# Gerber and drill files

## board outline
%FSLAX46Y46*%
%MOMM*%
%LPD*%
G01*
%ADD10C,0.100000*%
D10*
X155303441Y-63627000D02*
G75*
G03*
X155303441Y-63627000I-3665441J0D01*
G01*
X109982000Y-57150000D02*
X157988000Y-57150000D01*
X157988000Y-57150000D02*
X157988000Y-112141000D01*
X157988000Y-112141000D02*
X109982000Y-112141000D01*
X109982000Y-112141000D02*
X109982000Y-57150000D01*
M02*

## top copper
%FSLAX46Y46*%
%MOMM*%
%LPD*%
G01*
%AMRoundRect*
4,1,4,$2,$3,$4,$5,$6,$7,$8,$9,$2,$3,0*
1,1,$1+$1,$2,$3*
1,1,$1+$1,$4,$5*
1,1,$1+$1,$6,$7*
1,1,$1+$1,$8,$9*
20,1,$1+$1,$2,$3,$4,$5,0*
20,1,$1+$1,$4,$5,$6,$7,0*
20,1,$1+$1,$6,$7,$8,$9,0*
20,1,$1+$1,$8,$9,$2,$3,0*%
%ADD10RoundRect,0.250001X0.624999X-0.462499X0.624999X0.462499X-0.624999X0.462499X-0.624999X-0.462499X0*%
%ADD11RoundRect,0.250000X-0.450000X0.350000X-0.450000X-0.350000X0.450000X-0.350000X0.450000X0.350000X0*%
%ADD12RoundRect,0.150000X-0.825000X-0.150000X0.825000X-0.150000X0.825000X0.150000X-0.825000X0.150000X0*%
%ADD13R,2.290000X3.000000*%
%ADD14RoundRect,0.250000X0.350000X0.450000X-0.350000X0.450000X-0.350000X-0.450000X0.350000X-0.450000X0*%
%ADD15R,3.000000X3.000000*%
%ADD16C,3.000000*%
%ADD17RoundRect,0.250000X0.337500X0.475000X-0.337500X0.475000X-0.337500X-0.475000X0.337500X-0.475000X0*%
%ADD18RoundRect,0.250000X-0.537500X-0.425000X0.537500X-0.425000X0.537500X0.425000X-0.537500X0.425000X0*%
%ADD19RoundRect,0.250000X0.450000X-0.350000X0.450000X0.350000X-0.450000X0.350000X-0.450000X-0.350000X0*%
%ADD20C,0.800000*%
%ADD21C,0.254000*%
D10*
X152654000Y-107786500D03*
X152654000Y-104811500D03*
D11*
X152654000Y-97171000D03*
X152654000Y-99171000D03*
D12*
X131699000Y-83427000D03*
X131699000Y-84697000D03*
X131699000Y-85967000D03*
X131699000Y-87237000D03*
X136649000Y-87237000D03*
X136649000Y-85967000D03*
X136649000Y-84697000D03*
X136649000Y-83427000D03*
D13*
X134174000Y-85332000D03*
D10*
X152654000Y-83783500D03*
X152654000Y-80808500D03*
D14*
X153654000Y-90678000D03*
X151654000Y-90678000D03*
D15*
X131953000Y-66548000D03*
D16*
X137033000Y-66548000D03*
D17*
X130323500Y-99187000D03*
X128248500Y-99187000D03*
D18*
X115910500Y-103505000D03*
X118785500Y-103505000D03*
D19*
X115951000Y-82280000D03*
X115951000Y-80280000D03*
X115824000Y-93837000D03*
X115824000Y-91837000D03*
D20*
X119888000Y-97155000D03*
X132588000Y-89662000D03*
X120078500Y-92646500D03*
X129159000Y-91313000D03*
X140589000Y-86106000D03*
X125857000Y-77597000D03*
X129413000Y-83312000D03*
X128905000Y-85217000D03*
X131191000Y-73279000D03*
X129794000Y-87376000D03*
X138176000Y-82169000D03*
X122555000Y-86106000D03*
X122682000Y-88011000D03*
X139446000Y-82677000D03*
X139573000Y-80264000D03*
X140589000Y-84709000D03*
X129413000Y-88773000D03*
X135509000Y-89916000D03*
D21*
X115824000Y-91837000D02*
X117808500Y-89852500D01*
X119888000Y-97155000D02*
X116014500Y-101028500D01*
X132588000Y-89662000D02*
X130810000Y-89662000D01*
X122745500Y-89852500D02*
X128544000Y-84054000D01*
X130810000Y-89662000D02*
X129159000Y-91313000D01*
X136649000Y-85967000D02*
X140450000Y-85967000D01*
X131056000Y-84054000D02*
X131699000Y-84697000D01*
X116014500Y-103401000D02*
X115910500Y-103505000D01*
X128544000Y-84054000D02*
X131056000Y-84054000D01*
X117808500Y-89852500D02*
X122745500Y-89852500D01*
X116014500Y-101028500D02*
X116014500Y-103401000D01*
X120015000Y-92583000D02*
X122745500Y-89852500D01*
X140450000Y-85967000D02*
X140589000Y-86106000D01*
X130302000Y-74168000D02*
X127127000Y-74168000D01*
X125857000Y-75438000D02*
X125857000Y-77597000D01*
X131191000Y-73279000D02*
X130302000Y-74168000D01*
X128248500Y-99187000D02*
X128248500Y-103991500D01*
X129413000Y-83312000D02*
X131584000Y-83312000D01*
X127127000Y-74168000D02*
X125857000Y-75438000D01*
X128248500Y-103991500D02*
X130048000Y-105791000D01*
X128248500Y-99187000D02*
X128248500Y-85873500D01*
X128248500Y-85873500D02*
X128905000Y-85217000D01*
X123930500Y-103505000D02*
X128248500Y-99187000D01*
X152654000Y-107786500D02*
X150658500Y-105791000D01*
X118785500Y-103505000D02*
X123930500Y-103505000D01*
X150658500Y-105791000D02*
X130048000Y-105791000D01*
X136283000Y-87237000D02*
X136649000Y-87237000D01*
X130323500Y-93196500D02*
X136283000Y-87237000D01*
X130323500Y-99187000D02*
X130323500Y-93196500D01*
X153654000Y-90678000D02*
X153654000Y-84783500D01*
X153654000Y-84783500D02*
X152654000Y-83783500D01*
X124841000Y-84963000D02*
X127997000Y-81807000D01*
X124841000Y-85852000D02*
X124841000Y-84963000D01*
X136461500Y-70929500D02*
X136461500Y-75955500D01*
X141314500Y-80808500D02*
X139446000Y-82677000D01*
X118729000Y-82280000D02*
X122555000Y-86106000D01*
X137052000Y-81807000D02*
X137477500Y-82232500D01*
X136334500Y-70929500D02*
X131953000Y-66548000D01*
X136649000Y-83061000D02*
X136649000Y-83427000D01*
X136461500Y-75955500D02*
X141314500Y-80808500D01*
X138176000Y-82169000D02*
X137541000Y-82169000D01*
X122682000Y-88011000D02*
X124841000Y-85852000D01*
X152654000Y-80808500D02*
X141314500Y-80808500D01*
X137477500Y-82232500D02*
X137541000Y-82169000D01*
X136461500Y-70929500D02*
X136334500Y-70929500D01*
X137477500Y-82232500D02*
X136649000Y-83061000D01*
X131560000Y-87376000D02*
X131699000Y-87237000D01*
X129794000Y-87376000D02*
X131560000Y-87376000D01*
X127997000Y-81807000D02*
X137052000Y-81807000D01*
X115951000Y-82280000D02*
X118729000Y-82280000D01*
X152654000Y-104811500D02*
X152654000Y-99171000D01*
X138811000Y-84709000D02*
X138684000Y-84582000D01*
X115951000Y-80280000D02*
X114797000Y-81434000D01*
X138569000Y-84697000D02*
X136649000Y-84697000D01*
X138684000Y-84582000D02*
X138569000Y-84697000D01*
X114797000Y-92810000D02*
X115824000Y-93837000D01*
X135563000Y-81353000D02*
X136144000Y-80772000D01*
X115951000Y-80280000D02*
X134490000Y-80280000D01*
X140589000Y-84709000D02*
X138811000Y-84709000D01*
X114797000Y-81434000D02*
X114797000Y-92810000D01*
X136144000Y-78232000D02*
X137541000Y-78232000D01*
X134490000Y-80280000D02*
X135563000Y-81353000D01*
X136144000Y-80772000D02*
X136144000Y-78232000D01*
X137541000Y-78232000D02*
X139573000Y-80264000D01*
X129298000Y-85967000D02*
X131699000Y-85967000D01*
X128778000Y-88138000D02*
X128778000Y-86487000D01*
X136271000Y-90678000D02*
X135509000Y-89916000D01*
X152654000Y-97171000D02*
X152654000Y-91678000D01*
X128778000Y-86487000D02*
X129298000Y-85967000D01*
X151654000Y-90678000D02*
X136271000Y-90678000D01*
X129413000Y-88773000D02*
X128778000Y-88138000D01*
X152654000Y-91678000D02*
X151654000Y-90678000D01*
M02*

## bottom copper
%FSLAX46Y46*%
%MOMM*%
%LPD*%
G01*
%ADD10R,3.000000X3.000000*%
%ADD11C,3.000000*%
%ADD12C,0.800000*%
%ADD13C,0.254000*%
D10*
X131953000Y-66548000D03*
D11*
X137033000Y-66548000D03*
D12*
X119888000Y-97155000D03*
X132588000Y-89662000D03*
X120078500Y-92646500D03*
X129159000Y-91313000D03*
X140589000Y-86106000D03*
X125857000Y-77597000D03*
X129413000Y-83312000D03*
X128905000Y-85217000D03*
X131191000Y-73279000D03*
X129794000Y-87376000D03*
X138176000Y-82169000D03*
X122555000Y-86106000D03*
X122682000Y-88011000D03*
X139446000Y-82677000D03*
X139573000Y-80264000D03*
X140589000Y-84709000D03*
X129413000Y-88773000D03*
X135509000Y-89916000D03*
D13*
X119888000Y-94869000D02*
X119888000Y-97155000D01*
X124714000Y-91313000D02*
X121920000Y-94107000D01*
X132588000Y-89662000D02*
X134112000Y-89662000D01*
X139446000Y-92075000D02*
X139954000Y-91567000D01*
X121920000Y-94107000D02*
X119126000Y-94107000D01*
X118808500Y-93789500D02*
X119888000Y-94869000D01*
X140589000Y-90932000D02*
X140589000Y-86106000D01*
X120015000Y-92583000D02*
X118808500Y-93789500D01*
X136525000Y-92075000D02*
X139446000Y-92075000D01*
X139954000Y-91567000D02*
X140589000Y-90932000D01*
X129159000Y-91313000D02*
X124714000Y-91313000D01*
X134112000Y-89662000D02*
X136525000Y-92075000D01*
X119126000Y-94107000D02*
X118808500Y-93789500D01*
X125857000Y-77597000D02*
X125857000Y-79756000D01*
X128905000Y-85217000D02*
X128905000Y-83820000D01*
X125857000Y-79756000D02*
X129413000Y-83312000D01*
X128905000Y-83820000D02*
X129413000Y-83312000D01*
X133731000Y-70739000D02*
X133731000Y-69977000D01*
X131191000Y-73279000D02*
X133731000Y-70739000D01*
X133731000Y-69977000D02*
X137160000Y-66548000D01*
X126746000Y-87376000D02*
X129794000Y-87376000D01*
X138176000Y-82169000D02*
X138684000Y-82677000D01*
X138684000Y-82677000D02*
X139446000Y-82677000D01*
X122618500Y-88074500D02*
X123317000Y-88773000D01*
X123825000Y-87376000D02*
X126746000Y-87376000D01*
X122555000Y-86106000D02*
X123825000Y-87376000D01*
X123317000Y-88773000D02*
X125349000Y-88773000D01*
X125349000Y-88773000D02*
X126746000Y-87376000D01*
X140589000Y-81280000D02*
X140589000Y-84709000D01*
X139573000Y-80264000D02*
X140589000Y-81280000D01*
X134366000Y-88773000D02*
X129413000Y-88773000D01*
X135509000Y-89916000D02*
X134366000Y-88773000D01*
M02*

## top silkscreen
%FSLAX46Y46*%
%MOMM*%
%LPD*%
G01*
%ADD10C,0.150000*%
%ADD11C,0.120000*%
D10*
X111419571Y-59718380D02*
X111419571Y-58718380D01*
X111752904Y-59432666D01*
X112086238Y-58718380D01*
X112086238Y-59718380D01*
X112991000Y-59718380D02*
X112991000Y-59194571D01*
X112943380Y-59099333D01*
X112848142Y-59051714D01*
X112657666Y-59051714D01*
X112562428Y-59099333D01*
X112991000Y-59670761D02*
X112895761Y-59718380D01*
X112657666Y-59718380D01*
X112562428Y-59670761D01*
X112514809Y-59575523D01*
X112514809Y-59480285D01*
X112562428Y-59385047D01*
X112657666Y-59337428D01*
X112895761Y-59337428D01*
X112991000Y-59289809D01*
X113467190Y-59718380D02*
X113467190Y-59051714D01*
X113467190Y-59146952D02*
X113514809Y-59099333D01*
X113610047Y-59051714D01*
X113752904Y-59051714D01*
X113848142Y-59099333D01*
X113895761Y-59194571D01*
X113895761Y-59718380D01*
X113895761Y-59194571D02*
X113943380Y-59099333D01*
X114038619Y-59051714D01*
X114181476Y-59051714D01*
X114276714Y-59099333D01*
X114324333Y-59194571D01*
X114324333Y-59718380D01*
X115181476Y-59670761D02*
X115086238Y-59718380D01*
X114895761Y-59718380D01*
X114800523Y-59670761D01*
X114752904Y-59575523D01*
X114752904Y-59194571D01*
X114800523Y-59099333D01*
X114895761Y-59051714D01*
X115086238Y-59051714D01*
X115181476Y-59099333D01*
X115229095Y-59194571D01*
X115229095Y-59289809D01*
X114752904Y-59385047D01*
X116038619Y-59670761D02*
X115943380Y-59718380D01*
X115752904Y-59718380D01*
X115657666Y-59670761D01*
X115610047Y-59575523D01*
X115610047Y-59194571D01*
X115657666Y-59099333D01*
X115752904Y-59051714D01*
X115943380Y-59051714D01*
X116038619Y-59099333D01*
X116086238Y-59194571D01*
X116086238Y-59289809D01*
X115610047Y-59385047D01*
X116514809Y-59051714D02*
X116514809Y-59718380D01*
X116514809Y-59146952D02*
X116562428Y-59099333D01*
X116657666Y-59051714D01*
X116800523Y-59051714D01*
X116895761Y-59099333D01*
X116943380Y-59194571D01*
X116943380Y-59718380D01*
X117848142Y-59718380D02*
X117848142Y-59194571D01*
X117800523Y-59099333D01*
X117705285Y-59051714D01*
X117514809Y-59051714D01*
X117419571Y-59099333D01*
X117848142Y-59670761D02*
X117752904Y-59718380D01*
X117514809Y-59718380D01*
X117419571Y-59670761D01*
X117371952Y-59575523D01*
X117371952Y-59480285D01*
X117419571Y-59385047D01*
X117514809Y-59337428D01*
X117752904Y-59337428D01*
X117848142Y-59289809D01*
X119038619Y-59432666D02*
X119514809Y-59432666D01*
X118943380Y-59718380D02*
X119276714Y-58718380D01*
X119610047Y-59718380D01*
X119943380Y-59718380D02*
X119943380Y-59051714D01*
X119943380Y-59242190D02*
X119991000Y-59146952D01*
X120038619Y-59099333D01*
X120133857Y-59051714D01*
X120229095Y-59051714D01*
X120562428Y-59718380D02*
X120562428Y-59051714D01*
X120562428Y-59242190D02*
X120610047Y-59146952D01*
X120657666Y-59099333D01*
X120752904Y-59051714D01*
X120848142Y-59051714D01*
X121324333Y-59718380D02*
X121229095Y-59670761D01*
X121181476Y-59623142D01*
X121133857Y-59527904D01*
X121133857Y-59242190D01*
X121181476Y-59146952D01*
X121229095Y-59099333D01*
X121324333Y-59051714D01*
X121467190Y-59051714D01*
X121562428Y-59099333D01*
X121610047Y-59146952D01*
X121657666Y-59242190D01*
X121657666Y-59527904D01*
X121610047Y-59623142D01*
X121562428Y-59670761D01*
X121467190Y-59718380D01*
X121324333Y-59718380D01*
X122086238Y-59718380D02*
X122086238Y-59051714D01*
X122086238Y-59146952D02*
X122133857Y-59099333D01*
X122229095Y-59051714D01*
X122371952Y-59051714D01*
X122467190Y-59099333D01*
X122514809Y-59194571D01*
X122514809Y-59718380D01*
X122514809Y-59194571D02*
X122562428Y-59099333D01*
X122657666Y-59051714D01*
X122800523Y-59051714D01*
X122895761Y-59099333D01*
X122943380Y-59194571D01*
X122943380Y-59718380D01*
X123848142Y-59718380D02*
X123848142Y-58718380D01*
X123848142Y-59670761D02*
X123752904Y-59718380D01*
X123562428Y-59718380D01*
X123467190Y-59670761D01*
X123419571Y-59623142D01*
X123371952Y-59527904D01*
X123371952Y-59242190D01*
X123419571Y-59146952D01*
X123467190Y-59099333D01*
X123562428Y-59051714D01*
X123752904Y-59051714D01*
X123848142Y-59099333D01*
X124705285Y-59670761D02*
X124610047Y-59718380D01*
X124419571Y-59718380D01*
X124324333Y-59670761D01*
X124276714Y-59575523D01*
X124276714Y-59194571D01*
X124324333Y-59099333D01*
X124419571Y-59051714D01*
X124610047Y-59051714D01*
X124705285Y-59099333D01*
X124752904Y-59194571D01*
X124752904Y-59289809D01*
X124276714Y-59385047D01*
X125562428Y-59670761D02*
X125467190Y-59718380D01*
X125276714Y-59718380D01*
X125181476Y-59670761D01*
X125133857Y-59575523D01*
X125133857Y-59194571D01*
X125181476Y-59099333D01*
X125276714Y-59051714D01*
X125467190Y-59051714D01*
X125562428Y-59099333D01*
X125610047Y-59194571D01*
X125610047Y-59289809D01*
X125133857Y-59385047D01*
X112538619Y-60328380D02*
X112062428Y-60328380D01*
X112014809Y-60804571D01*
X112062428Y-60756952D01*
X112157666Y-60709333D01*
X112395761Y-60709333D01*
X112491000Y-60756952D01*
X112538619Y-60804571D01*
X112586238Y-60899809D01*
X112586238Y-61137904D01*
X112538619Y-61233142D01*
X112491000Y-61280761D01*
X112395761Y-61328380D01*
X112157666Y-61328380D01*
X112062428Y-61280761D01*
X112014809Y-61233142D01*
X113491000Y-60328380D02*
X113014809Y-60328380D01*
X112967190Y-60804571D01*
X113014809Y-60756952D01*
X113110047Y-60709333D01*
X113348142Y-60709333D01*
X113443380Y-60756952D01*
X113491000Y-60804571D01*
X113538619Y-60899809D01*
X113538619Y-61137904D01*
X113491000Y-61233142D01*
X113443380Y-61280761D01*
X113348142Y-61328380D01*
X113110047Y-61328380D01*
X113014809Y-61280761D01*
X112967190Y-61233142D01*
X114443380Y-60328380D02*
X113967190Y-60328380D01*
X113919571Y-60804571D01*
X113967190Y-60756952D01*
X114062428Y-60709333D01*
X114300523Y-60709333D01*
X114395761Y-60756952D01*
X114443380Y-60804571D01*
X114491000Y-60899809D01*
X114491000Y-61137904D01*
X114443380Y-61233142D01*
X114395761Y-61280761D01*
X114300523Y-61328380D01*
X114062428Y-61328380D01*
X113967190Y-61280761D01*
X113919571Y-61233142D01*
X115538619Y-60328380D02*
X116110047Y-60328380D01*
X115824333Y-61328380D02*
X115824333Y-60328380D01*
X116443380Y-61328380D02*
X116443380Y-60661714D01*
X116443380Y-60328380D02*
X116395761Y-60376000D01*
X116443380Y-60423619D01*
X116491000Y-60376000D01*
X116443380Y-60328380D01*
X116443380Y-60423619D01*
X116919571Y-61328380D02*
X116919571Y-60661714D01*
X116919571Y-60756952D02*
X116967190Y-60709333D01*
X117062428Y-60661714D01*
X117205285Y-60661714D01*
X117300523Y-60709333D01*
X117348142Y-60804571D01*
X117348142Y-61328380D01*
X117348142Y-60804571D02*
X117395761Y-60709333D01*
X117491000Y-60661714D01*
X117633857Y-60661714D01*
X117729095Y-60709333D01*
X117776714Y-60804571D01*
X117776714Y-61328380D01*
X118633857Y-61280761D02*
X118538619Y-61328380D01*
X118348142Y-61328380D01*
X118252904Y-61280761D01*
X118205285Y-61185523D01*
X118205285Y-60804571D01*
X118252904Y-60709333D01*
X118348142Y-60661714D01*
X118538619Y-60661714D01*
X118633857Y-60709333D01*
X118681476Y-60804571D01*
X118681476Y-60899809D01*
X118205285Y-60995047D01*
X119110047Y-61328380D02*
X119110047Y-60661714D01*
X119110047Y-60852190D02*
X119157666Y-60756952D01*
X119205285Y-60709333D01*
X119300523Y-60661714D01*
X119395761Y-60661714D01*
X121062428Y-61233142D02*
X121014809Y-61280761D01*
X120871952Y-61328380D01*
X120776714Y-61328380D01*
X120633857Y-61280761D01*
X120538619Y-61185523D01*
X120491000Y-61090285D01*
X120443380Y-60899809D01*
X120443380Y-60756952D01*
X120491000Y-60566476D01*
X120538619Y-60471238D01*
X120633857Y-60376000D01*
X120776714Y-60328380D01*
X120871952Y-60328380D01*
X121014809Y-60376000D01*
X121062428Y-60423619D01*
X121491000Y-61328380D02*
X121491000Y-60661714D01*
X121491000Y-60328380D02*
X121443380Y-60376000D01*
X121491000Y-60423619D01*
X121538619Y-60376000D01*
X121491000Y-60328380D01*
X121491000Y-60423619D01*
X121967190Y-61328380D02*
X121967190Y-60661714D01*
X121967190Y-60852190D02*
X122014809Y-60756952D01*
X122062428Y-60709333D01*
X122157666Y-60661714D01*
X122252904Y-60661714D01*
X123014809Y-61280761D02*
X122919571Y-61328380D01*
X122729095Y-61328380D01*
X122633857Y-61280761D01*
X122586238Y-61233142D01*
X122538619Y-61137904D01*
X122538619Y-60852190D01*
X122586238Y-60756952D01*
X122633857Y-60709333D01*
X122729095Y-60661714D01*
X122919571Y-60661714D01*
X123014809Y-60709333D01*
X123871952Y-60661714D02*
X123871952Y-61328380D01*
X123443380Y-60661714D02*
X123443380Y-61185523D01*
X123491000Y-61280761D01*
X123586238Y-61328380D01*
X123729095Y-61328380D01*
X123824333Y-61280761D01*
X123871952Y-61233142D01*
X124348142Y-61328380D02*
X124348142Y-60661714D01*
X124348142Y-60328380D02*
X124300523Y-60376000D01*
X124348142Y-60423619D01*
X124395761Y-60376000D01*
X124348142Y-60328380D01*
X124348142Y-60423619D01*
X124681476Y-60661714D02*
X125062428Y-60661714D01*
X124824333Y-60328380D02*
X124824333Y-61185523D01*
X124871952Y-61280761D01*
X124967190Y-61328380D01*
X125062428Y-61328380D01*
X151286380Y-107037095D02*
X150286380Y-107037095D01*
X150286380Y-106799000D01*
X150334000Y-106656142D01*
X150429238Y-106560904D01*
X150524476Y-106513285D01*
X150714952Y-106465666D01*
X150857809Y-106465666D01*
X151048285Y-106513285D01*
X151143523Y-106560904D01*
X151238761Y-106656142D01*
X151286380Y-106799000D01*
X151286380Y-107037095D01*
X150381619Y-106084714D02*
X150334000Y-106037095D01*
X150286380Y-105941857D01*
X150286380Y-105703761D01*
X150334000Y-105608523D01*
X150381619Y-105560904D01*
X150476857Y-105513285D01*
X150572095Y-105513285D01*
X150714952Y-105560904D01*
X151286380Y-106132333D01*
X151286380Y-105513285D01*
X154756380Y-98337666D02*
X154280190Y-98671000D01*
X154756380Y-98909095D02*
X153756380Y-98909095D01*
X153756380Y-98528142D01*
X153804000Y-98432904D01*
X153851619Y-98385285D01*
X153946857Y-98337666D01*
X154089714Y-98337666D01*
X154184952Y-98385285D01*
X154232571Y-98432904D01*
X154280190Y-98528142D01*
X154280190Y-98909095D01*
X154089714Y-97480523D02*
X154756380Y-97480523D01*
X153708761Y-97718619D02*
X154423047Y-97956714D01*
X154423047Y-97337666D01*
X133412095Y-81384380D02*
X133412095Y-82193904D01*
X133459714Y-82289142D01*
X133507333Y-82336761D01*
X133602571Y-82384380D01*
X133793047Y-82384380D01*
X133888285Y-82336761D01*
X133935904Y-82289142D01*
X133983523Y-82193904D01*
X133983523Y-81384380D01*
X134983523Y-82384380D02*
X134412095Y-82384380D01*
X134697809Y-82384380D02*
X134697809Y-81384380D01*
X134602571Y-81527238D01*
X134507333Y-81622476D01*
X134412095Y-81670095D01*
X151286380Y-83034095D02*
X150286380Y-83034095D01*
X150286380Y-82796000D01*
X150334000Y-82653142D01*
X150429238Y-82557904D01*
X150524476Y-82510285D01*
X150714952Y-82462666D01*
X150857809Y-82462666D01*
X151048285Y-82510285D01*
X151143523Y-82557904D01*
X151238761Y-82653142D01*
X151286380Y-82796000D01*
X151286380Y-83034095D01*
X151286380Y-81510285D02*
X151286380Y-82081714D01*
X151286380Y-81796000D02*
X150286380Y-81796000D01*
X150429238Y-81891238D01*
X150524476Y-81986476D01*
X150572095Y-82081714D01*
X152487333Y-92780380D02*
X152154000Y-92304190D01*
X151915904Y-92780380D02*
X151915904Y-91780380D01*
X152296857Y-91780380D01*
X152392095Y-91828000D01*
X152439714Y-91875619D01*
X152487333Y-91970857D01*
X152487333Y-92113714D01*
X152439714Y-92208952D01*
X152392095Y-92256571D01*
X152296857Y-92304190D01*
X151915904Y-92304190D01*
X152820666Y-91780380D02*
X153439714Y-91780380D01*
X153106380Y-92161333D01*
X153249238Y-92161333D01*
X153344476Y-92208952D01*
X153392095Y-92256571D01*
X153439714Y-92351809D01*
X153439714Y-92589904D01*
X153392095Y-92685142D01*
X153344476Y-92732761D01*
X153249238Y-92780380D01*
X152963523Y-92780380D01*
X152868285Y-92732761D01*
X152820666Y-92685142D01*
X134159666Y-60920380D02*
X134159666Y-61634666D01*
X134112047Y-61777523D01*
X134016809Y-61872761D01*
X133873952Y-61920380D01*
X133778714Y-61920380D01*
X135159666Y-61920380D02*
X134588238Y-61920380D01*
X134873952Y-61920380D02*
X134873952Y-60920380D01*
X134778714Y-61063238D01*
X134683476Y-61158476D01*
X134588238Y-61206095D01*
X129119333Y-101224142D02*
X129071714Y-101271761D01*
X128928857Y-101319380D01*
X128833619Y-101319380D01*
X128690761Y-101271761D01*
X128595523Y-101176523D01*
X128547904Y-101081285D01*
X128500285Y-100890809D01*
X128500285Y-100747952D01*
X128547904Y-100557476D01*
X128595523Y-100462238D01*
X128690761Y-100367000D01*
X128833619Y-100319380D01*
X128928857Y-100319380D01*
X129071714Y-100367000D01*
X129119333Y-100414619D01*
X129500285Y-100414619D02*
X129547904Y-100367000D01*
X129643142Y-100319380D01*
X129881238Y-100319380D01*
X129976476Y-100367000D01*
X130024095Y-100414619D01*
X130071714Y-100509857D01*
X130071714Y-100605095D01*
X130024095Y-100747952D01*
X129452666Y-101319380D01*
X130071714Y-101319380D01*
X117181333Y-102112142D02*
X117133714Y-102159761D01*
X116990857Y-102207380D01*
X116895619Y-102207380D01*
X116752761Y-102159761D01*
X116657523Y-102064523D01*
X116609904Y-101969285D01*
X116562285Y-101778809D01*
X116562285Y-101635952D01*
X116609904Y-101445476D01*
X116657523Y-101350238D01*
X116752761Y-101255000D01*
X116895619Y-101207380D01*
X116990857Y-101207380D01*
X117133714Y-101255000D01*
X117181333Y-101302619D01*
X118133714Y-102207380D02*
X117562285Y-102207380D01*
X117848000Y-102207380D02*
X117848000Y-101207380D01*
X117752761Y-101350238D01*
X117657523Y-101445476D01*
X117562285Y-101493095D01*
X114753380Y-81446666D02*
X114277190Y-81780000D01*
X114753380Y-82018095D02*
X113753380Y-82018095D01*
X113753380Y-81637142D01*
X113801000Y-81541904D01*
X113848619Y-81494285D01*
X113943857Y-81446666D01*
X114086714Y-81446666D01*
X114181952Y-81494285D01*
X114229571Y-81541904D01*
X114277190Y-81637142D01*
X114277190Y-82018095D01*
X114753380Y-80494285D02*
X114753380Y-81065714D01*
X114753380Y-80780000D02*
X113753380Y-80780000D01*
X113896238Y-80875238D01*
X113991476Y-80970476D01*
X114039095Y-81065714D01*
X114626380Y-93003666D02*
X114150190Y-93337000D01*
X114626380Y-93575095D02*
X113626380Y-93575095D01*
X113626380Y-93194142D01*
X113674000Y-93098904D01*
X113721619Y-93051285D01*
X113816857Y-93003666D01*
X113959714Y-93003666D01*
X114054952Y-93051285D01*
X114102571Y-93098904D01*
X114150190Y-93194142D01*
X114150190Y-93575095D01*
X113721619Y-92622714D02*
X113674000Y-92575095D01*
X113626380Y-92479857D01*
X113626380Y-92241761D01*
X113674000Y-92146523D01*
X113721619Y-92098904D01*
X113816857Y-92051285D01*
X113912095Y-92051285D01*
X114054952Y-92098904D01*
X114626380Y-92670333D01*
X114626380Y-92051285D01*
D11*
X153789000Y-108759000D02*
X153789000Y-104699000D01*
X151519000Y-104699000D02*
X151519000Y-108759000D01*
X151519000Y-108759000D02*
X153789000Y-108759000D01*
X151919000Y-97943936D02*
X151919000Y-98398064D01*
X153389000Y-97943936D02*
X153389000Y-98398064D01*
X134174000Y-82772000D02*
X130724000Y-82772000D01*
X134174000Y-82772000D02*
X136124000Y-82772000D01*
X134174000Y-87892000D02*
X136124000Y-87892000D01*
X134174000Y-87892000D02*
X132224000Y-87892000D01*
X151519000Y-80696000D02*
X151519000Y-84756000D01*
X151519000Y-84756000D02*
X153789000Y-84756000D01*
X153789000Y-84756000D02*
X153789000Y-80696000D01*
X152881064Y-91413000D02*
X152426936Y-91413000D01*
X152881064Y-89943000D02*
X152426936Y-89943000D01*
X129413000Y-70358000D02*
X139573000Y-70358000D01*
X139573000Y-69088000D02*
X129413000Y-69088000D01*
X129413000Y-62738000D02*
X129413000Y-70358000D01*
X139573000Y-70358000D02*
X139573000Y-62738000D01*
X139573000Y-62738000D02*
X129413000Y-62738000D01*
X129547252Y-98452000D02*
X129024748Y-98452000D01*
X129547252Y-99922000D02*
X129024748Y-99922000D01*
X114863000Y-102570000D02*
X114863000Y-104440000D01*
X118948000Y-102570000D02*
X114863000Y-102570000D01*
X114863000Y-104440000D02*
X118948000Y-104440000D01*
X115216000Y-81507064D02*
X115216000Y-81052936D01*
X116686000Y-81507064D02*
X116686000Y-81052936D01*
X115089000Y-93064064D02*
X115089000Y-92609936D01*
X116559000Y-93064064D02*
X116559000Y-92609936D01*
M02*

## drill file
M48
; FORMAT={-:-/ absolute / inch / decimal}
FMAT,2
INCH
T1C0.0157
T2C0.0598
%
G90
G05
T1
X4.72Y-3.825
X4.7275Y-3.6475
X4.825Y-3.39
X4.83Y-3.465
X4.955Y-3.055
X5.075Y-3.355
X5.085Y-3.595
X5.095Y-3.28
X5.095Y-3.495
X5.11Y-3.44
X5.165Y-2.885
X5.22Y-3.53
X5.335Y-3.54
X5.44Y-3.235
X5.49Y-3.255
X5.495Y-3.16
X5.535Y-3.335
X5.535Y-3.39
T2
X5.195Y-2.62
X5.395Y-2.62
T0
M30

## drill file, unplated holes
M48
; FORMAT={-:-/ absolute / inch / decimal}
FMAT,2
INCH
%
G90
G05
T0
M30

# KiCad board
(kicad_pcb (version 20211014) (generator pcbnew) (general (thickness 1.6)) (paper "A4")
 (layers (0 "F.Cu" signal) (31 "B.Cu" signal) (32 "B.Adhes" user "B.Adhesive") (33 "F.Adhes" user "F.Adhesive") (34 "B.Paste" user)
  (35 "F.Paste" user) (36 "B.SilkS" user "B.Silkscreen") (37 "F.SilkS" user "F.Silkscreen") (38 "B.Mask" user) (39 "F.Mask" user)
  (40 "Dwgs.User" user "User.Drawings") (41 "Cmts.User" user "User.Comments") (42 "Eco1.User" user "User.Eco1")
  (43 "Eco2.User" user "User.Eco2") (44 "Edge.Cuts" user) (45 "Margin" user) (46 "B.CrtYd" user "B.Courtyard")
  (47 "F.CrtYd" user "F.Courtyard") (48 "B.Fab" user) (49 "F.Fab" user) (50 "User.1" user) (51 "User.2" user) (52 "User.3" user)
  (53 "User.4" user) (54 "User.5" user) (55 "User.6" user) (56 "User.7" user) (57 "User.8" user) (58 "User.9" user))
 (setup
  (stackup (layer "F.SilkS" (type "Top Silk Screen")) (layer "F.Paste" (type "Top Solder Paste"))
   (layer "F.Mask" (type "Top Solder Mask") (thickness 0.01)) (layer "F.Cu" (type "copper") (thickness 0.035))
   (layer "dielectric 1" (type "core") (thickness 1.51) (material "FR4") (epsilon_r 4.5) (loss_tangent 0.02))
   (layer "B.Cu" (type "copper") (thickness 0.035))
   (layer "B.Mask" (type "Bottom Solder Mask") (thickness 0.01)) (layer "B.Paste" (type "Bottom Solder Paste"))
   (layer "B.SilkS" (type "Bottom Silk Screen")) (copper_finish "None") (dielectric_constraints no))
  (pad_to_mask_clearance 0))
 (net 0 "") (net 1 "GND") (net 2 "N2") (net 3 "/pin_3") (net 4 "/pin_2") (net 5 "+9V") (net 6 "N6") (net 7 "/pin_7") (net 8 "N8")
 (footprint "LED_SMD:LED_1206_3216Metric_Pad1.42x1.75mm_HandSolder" (layer "F.Cu") (at 152.654 106.299 90)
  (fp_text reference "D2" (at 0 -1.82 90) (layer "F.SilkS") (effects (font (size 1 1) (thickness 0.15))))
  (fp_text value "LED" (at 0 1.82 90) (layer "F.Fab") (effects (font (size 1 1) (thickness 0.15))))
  (fp_line (start -2.46 1.135) (end 1.6 1.135) (layer "F.SilkS") (width 0.12))
  (fp_line (start 1.6 -1.135) (end -2.46 -1.135) (layer "F.SilkS") (width 0.12))
  (fp_line (start -2.46 -1.135) (end -2.46 1.135) (layer "F.SilkS") (width 0.12))
  (pad "1" smd roundrect (at -1.4875 0 90) (size 1.425 1.75) (layers "F.Cu" "F.Paste" "F.Mask") (roundrect_rratio 0.1754392982)
   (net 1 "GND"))
  (pad "2" smd roundrect (at 1.4875 0 90) (size 1.425 1.75) (layers "F.Cu" "F.Paste" "F.Mask") (roundrect_rratio 0.1754392982) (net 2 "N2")))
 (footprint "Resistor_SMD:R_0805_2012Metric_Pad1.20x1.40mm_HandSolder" (layer "F.Cu") (at 152.654 98.171 -90)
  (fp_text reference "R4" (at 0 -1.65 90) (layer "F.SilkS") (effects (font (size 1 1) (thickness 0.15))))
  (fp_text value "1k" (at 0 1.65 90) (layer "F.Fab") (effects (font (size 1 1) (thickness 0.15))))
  (fp_line (start -0.227064 0.735) (end 0.227064 0.735) (layer "F.SilkS") (width 0.12))
  (fp_line (start -0.227064 -0.735) (end 0.227064 -0.735) (layer "F.SilkS") (width 0.12))
  (pad "1" smd roundrect (at -1 0 270) (size 1.2 1.4) (layers "F.Cu" "F.Paste" "F.Mask") (roundrect_rratio 0.2083333333) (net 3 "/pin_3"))
  (pad "2" smd roundrect (at 1 0 270) (size 1.2 1.4) (layers "F.Cu" "F.Paste" "F.Mask") (roundrect_rratio 0.2083333333) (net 2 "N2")))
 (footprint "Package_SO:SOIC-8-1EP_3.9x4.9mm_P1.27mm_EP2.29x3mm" (layer "F.Cu") (at 134.174 85.332)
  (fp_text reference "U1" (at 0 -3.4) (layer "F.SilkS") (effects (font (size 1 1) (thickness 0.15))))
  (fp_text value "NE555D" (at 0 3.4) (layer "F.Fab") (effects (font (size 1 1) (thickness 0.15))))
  (fp_line (start 0 -2.56) (end -3.45 -2.56) (layer "F.SilkS") (width 0.12))
  (fp_line (start 0 -2.56) (end 1.95 -2.56) (layer "F.SilkS") (width 0.12))
  (fp_line (start 0 2.56) (end 1.95 2.56) (layer "F.SilkS") (width 0.12))
  (fp_line (start 0 2.56) (end -1.95 2.56) (layer "F.SilkS") (width 0.12))
  (pad "" smd roundrect (at 0.57 -0.75) (size 0.92 1.21) (layers "F.Paste") (roundrect_rratio 0.25))
  (pad "" smd roundrect (at -0.57 -0.75) (size 0.92 1.21) (layers "F.Paste") (roundrect_rratio 0.25))
  (pad "" smd roundrect (at -0.57 0.75) (size 0.92 1.21) (layers "F.Paste") (roundrect_rratio 0.25))
  (pad "" smd roundrect (at 0.57 0.75) (size 0.92 1.21) (layers "F.Paste") (roundrect_rratio 0.25))
  (pad "1" smd roundrect (at -2.475 -1.905) (size 1.95 0.6) (layers "F.Cu" "F.Paste" "F.Mask") (roundrect_rratio 0.25) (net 1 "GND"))
  (pad "2" smd roundrect (at -2.475 -0.635) (size 1.95 0.6) (layers "F.Cu" "F.Paste" "F.Mask") (roundrect_rratio 0.25) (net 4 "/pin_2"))
  (pad "3" smd roundrect (at -2.475 0.635) (size 1.95 0.6) (layers "F.Cu" "F.Paste" "F.Mask") (roundrect_rratio 0.25) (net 3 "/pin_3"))
  (pad "4" smd roundrect (at -2.475 1.905) (size 1.95 0.6) (layers "F.Cu" "F.Paste" "F.Mask") (roundrect_rratio 0.25) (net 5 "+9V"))
  (pad "5" smd roundrect (at 2.475 1.905) (size 1.95 0.6) (layers "F.Cu" "F.Paste" "F.Mask") (roundrect_rratio 0.25) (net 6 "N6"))
  (pad "6" smd roundrect (at 2.475 0.635) (size 1.95 0.6) (layers "F.Cu" "F.Paste" "F.Mask") (roundrect_rratio 0.25) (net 4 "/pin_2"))
  (pad "7" smd roundrect (at 2.475 -0.635) (size 1.95 0.6) (layers "F.Cu" "F.Paste" "F.Mask") (roundrect_rratio 0.25) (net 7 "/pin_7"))
  (pad "8" smd roundrect (at 2.475 -1.905) (size 1.95 0.6) (layers "F.Cu" "F.Paste" "F.Mask") (roundrect_rratio 0.25) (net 5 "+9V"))
  (pad "9" smd rect (at 0 0) (size 2.29 3) (layers "F.Cu" "F.Mask")))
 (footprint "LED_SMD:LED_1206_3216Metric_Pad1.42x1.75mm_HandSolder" (layer "F.Cu") (at 152.654 82.296 90)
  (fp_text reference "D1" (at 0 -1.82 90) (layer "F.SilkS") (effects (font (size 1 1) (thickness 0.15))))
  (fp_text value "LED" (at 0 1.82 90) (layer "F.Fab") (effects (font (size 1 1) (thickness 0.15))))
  (fp_line (start 1.6 -1.135) (end -2.46 -1.135) (layer "F.SilkS") (width 0.12))
  (fp_line (start -2.46 -1.135) (end -2.46 1.135) (layer "F.SilkS") (width 0.12))
  (fp_line (start -2.46 1.135) (end 1.6 1.135) (layer "F.SilkS") (width 0.12))
  (pad "1" smd roundrect (at -1.4875 0 90) (size 1.425 1.75) (layers "F.Cu" "F.Paste" "F.Mask") (roundrect_rratio 0.1754392982) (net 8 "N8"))
  (pad "2" smd roundrect (at 1.4875 0 90) (size 1.425 1.75) (layers "F.Cu" "F.Paste" "F.Mask") (roundrect_rratio 0.1754392982) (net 5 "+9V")))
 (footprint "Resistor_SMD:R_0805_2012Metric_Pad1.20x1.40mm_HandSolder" (layer "F.Cu") (at 152.654 90.678 180)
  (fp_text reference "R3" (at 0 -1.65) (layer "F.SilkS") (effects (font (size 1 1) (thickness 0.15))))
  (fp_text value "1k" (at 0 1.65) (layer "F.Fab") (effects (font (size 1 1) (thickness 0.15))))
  (fp_line (start -0.227064 -0.735) (end 0.227064 -0.735) (layer "F.SilkS") (width 0.12))
  (fp_line (start -0.227064 0.735) (end 0.227064 0.735) (layer "F.SilkS") (width 0.12))
  (pad "1" smd roundrect (at -1 0 180) (size 1.2 1.4) (layers "F.Cu" "F.Paste" "F.Mask") (roundrect_rratio 0.2083333333) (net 8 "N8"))
  (pad "2" smd roundrect (at 1 0 180) (size 1.2 1.4) (layers "F.Cu" "F.Paste" "F.Mask") (roundrect_rratio 0.2083333333) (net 3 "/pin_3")))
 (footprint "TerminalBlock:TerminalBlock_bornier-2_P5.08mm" (layer "F.Cu") (at 131.953 66.548)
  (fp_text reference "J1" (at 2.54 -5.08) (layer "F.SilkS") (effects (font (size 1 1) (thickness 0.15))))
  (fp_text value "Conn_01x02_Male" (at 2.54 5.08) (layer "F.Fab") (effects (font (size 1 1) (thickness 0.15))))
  (fp_line (start -2.54 3.81) (end 7.62 3.81) (layer "F.SilkS") (width 0.12))
  (fp_line (start 7.62 2.54) (end -2.54 2.54) (layer "F.SilkS") (width 0.12))
  (fp_line (start -2.54 -3.81) (end -2.54 3.81) (layer "F.SilkS") (width 0.12))
  (fp_line (start 7.62 3.81) (end 7.62 -3.81) (layer "F.SilkS") (width 0.12))
  (fp_line (start 7.62 -3.81) (end -2.54 -3.81) (layer "F.SilkS") (width 0.12))
  (pad "1" thru_hole rect (at 0 0) (size 3 3) (drill 1.52) (layers *.Cu *.Mask) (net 5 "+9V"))
  (pad "2" thru_hole circle (at 5.08 0) (size 3 3) (drill 1.52) (layers *.Cu *.Mask) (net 1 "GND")))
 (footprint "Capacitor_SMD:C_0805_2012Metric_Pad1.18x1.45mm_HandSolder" (layer "F.Cu") (at 129.286 99.187 180)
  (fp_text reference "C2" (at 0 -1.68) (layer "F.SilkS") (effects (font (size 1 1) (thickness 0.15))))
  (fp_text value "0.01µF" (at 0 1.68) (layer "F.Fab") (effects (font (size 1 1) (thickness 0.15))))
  (fp_line (start -0.261252 0.735) (end 0.261252 0.735) (layer "F.SilkS") (width 0.12))
  (fp_line (start -0.261252 -0.735) (end 0.261252 -0.735) (layer "F.SilkS") (width 0.12))
  (pad "1" smd roundrect (at -1.0375 0 180) (size 1.175 1.45) (layers "F.Cu" "F.Paste" "F.Mask") (roundrect_rratio 0.2127659574)
   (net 6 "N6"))
  (pad "2" smd roundrect (at 1.0375 0 180) (size 1.175 1.45) (layers "F.Cu" "F.Paste" "F.Mask") (roundrect_rratio 0.2127659574)
   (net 1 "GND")))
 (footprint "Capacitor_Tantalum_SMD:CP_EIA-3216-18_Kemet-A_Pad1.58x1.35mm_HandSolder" (layer "F.Cu") (at 117.348 103.505)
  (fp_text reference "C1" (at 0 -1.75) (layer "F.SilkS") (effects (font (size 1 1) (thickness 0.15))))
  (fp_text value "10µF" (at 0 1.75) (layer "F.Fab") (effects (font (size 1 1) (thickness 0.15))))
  (fp_line (start -2.485 -0.935) (end -2.485 0.935) (layer "F.SilkS") (width 0.12))
  (fp_line (start 1.6 -0.935) (end -2.485 -0.935) (layer "F.SilkS") (width 0.12))
  (fp_line (start -2.485 0.935) (end 1.6 0.935) (layer "F.SilkS") (width 0.12))
  (pad "1" smd roundrect (at -1.4375 0) (size 1.575 1.35) (layers "F.Cu" "F.Paste" "F.Mask") (roundrect_rratio 0.1851851852)
   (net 4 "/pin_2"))
  (pad "2" smd roundrect (at 1.4375 0) (size 1.575 1.35) (layers "F.Cu" "F.Paste" "F.Mask") (roundrect_rratio 0.1851851852) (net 1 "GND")))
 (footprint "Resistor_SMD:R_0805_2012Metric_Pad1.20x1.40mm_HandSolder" (layer "F.Cu") (at 115.951 81.28 90)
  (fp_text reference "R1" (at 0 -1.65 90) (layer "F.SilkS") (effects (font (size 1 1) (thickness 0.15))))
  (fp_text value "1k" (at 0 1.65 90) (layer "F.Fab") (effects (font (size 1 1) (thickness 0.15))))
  (fp_line (start -0.227064 -0.735) (end 0.227064 -0.735) (layer "F.SilkS") (width 0.12))
  (fp_line (start -0.227064 0.735) (end 0.227064 0.735) (layer "F.SilkS") (width 0.12))
  (pad "1" smd roundrect (at -1 0 90) (size 1.2 1.4) (layers "F.Cu" "F.Paste" "F.Mask") (roundrect_rratio 0.2083333333) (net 5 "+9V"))
  (pad "2" smd roundrect (at 1 0 90) (size 1.2 1.4) (layers "F.Cu" "F.Paste" "F.Mask") (roundrect_rratio 0.2083333333) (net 7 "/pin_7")))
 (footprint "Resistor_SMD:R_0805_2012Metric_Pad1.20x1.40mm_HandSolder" (layer "F.Cu") (at 115.824 92.837 90)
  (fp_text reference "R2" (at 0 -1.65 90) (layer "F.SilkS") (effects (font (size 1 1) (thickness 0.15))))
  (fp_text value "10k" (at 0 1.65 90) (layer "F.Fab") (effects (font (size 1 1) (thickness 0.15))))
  (fp_line (start -0.227064 -0.735) (end 0.227064 -0.735) (layer "F.SilkS") (width 0.12))
  (fp_line (start -0.227064 0.735) (end 0.227064 0.735) (layer "F.SilkS") (width 0.12))
  (pad "1" smd roundrect (at -1 0 90) (size 1.2 1.4) (layers "F.Cu" "F.Paste" "F.Mask") (roundrect_rratio 0.2083333333) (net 7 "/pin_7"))
  (pad "2" smd roundrect (at 1 0 90) (size 1.2 1.4) (layers "F.Cu" "F.Paste" "F.Mask") (roundrect_rratio 0.2083333333) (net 4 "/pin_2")))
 (gr_circle (center 151.638 63.627) (end 152.527 60.071) (layer "Edge.Cuts") (width 0.1) (fill none))
 (gr_rect (start 109.982 57.15) (end 157.988 112.141) (layer "Edge.Cuts") (width 0.1) (fill none))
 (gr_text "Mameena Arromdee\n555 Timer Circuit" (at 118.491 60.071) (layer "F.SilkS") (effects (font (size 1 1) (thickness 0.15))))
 (segment (start 115.824 91.837) (end 117.8085 89.8525) (width 0.254) (layer "F.Cu") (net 4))
 (segment (start 119.888 97.155) (end 116.0145 101.0285) (width 0.254) (layer "F.Cu") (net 4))
 (segment (start 132.588 89.662) (end 130.81 89.662) (width 0.254) (layer "F.Cu") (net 4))
 (segment (start 122.7455 89.8525) (end 128.544 84.054) (width 0.254) (layer "F.Cu") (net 4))
 (segment (start 130.81 89.662) (end 129.159 91.313) (width 0.254) (layer "F.Cu") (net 4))
 (segment (start 136.649 85.967) (end 140.45 85.967) (width 0.254) (layer "F.Cu") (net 4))
 (segment (start 131.056 84.054) (end 131.699 84.697) (width 0.254) (layer "F.Cu") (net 4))
 (segment (start 116.0145 103.401) (end 115.9105 103.505) (width 0.254) (layer "F.Cu") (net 4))
 (segment (start 128.544 84.054) (end 131.056 84.054) (width 0.254) (layer "F.Cu") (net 4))
 (segment (start 117.8085 89.8525) (end 122.7455 89.8525) (width 0.254) (layer "F.Cu") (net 4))
 (segment (start 116.0145 101.0285) (end 116.0145 103.401) (width 0.254) (layer "F.Cu") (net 4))
 (segment (start 120.015 92.583) (end 122.7455 89.8525) (width 0.254) (layer "F.Cu") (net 4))
 (segment (start 140.45 85.967) (end 140.589 86.106) (width 0.254) (layer "F.Cu") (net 4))
 (via (at 119.888 97.155) (size 0.8) (drill 0.4) (layers "F.Cu" "B.Cu") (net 4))
 (via (at 132.588 89.662) (size 0.8) (drill 0.4) (layers "F.Cu" "B.Cu") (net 4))
 (via (at 120.0785 92.6465) (size 0.8) (drill 0.4) (layers "F.Cu" "B.Cu") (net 4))
 (via (at 129.159 91.313) (size 0.8) (drill 0.4) (layers "F.Cu" "B.Cu") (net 4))
 (via (at 140.589 86.106) (size 0.8) (drill 0.4) (layers "F.Cu" "B.Cu") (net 4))
 (segment (start 119.888 94.869) (end 119.888 97.155) (width 0.254) (layer "B.Cu") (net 4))
 (segment (start 124.714 91.313) (end 121.92 94.107) (width 0.254) (layer "B.Cu") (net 4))
 (segment (start 132.588 89.662) (end 134.112 89.662) (width 0.254) (layer "B.Cu") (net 4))
 (segment (start 139.446 92.075) (end 139.954 91.567) (width 0.254) (layer "B.Cu") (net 4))
 (segment (start 121.92 94.107) (end 119.126 94.107) (width 0.254) (layer "B.Cu") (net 4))
 (segment (start 118.8085 93.7895) (end 119.888 94.869) (width 0.254) (layer "B.Cu") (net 4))
 (segment (start 140.589 90.932) (end 140.589 86.106) (width 0.254) (layer "B.Cu") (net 4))
 (segment (start 120.015 92.583) (end 118.8085 93.7895) (width 0.254) (layer "B.Cu") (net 4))
 (segment (start 136.525 92.075) (end 139.446 92.075) (width 0.254) (layer "B.Cu") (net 4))
 (segment (start 139.954 91.567) (end 140.589 90.932) (width 0.254) (layer "B.Cu") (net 4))
 (segment (start 129.159 91.313) (end 124.714 91.313) (width 0.254) (layer "B.Cu") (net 4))
 (segment (start 134.112 89.662) (end 136.525 92.075) (width 0.254) (layer "B.Cu") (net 4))
 (segment (start 119.126 94.107) (end 118.8085 93.7895) (width 0.254) (layer "B.Cu") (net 4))
 (segment (start 130.302 74.168) (end 127.127 74.168) (width 0.254) (layer "F.Cu") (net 1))
 (segment (start 125.857 75.438) (end 125.857 77.597) (width 0.254) (layer "F.Cu") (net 1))
 (segment (start 131.191 73.279) (end 130.302 74.168) (width 0.254) (layer "F.Cu") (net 1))
 (segment (start 128.2485 99.187) (end 128.2485 103.9915) (width 0.254) (layer "F.Cu") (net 1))
 (segment (start 129.413 83.312) (end 131.584 83.312) (width 0.254) (layer "F.Cu") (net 1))
 (segment (start 127.127 74.168) (end 125.857 75.438) (width 0.254) (layer "F.Cu") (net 1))
 (segment (start 128.2485 103.9915) (end 130.048 105.791) (width 0.254) (layer "F.Cu") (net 1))
 (segment (start 128.2485 99.187) (end 128.2485 85.8735) (width 0.254) (layer "F.Cu") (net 1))
 (segment (start 128.2485 85.8735) (end 128.905 85.217) (width 0.254) (layer "F.Cu") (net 1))
 (segment (start 123.9305 103.505) (end 128.2485 99.187) (width 0.254) (layer "F.Cu") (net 1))
 (segment (start 152.654 107.7865) (end 150.6585 105.791) (width 0.254) (layer "F.Cu") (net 1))
 (segment (start 118.7855 103.505) (end 123.9305 103.505) (width 0.254) (layer "F.Cu") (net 1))
 (segment (start 150.6585 105.791) (end 130.048 105.791) (width 0.254) (layer "F.Cu") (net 1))
 (via (at 125.857 77.597) (size 0.8) (drill 0.4) (layers "F.Cu" "B.Cu") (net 1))
 (via (at 129.413 83.312) (size 0.8) (drill 0.4) (layers "F.Cu" "B.Cu") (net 1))
 (via (at 128.905 85.217) (size 0.8) (drill 0.4) (layers "F.Cu" "B.Cu") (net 1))
 (via (at 131.191 73.279) (size 0.8) (drill 0.4) (layers "F.Cu" "B.Cu") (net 1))
 (segment (start 125.857 77.597) (end 125.857 79.756) (width 0.254) (layer "B.Cu") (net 1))
 (segment (start 128.905 85.217) (end 128.905 83.82) (width 0.254) (layer "B.Cu") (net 1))
 (segment (start 125.857 79.756) (end 129.413 83.312) (width 0.254) (layer "B.Cu") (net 1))
 (segment (start 128.905 83.82) (end 129.413 83.312) (width 0.254) (layer "B.Cu") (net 1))
 (segment (start 133.731 70.739) (end 133.731 69.977) (width 0.254) (layer "B.Cu") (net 1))
 (segment (start 131.191 73.279) (end 133.731 70.739) (width 0.254) (layer "B.Cu") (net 1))
 (segment (start 133.731 69.977) (end 137.16 66.548) (width 0.254) (layer "B.Cu") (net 1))
 (segment (start 136.283 87.237) (end 136.649 87.237) (width 0.254) (layer "F.Cu") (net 6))
 (segment (start 130.3235 93.1965) (end 136.283 87.237) (width 0.254) (layer "F.Cu") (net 6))
 (segment (start 130.3235 99.187) (end 130.3235 93.1965) (width 0.254) (layer "F.Cu") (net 6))
 (segment (start 153.654 90.678) (end 153.654 84.7835) (width 0.254) (layer "F.Cu") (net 8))
 (segment (start 153.654 84.7835) (end 152.654 83.7835) (width 0.254) (layer "F.Cu") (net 8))
 (segment (start 124.841 84.963) (end 127.997 81.807) (width 0.254) (layer "F.Cu") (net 5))
 (segment (start 124.841 85.852) (end 124.841 84.963) (width 0.254) (layer "F.Cu") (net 5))
 (segment (start 136.4615 70.9295) (end 136.4615 75.9555) (width 0.254) (layer "F.Cu") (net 5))
 (segment (start 141.3145 80.8085) (end 139.446 82.677) (width 0.254) (layer "F.Cu") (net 5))
 (segment (start 118.729 82.28) (end 122.555 86.106) (width 0.254) (layer "F.Cu") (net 5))
 (segment (start 137.052 81.807) (end 137.4775 82.2325) (width 0.254) (layer "F.Cu") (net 5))
 (segment (start 136.3345 70.9295) (end 131.953 66.548) (width 0.254) (layer "F.Cu") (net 5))
 (segment (start 136.649 83.061) (end 136.649 83.427) (width 0.254) (layer "F.Cu") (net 5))
 (segment (start 136.4615 75.9555) (end 141.3145 80.8085) (width 0.254) (layer "F.Cu") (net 5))
 (segment (start 138.176 82.169) (end 137.541 82.169) (width 0.254) (layer "F.Cu") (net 5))
 (segment (start 122.682 88.011) (end 124.841 85.852) (width 0.254) (layer "F.Cu") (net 5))
 (segment (start 152.654 80.8085) (end 141.3145 80.8085) (width 0.254) (layer "F.Cu") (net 5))
 (segment (start 137.4775 82.2325) (end 137.541 82.169) (width 0.254) (layer "F.Cu") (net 5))
 (segment (start 136.4615 70.9295) (end 136.3345 70.9295) (width 0.254) (layer "F.Cu") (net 5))
 (segment (start 137.4775 82.2325) (end 136.649 83.061) (width 0.254) (layer "F.Cu") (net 5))
 (segment (start 131.56 87.376) (end 131.699 87.237) (width 0.254) (layer "F.Cu") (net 5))
 (segment (start 129.794 87.376) (end 131.56 87.376) (width 0.254) (layer "F.Cu") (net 5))
 (segment (start 127.997 81.807) (end 137.052 81.807) (width 0.254) (layer "F.Cu") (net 5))
 (segment (start 115.951 82.28) (end 118.729 82.28) (width 0.254) (layer "F.Cu") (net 5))
 (via (at 129.794 87.376) (size 0.8) (drill 0.4) (layers "F.Cu" "B.Cu") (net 5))
 (via (at 138.176 82.169) (size 0.8) (drill 0.4) (layers "F.Cu" "B.Cu") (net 5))
 (via (at 122.555 86.106) (size 0.8) (drill 0.4) (layers "F.Cu" "B.Cu") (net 5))
 (via (at 122.682 88.011) (size 0.8) (drill 0.4) (layers "F.Cu" "B.Cu") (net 5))
 (via (at 139.446 82.677) (size 0.8) (drill 0.4) (layers "F.Cu" "B.Cu") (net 5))
 (segment (start 126.746 87.376) (end 129.794 87.376) (width 0.254) (layer "B.Cu") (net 5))
 (segment (start 138.176 82.169) (end 138.684 82.677) (width 0.254) (layer "B.Cu") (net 5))
 (segment (start 138.684 82.677) (end 139.446 82.677) (width 0.254) (layer "B.Cu") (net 5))
 (segment (start 122.6185 88.0745) (end 123.317 88.773) (width 0.254) (layer "B.Cu") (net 5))
 (segment (start 123.825 87.376) (end 126.746 87.376) (width 0.254) (layer "B.Cu") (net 5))
 (segment (start 122.555 86.106) (end 123.825 87.376) (width 0.254) (layer "B.Cu") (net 5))
 (segment (start 123.317 88.773) (end 125.349 88.773) (width 0.254) (layer "B.Cu") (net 5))
 (segment (start 125.349 88.773) (end 126.746 87.376) (width 0.254) (layer "B.Cu") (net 5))
 (segment (start 152.654 104.8115) (end 152.654 99.171) (width 0.254) (layer "F.Cu") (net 2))
 (segment (start 138.811 84.709) (end 138.684 84.582) (width 0.254) (layer "F.Cu") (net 7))
 (segment (start 115.951 80.28) (end 114.797 81.434) (width 0.254) (layer "F.Cu") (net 7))
 (segment (start 138.569 84.697) (end 136.649 84.697) (width 0.254) (layer "F.Cu") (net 7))
 (segment (start 138.684 84.582) (end 138.569 84.697) (width 0.254) (layer "F.Cu") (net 7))
 (segment (start 114.797 92.81) (end 115.824 93.837) (width 0.254) (layer "F.Cu") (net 7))
 (segment (start 135.563 81.353) (end 136.144 80.772) (width 0.254) (layer "F.Cu") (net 7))
 (segment (start 115.951 80.28) (end 134.49 80.28) (width 0.254) (layer "F.Cu") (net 7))
 (segment (start 140.589 84.709) (end 138.811 84.709) (width 0.254) (layer "F.Cu") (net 7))
 (segment (start 114.797 81.434) (end 114.797 92.81) (width 0.254) (layer "F.Cu") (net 7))
 (segment (start 136.144 78.232) (end 137.541 78.232) (width 0.254) (layer "F.Cu") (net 7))
 (segment (start 134.49 80.28) (end 135.563 81.353) (width 0.254) (layer "F.Cu") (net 7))
 (segment (start 136.144 80.772) (end 136.144 78.232) (width 0.254) (layer "F.Cu") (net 7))
 (segment (start 137.541 78.232) (end 139.573 80.264) (width 0.254) (layer "F.Cu") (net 7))
 (via (at 139.573 80.264) (size 0.8) (drill 0.4) (layers "F.Cu" "B.Cu") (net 7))
 (via (at 140.589 84.709) (size 0.8) (drill 0.4) (layers "F.Cu" "B.Cu") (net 7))
 (segment (start 140.589 81.28) (end 140.589 84.709) (width 0.254) (layer "B.Cu") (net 7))
 (segment (start 139.573 80.264) (end 140.589 81.28) (width 0.254) (layer "B.Cu") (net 7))
 (segment (start 129.298 85.967) (end 131.699 85.967) (width 0.254) (layer "F.Cu") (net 3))
 (segment (start 128.778 88.138) (end 128.778 86.487) (width 0.254) (layer "F.Cu") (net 3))
 (segment (start 136.271 90.678) (end 135.509 89.916) (width 0.254) (layer "F.Cu") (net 3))
 (segment (start 152.654 97.171) (end 152.654 91.678) (width 0.254) (layer "F.Cu") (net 3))
 (segment (start 128.778 86.487) (end 129.298 85.967) (width 0.254) (layer "F.Cu") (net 3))
 (segment (start 151.654 90.678) (end 136.271 90.678) (width 0.254) (layer "F.Cu") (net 3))
 (segment (start 129.413 88.773) (end 128.778 88.138) (width 0.254) (layer "F.Cu") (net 3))
 (segment (start 152.654 91.678) (end 151.654 90.678) (width 0.254) (layer "F.Cu") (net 3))
 (via (at 129.413 88.773) (size 0.8) (drill 0.4) (layers "F.Cu" "B.Cu") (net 3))
 (via (at 135.509 89.916) (size 0.8) (drill 0.4) (layers "F.Cu" "B.Cu") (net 3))
 (segment (start 134.366 88.773) (end 129.413 88.773) (width 0.254) (layer "B.Cu") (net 3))
 (segment (start 135.509 89.916) (end 134.366 88.773) (width 0.254) (layer "B.Cu") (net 3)))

